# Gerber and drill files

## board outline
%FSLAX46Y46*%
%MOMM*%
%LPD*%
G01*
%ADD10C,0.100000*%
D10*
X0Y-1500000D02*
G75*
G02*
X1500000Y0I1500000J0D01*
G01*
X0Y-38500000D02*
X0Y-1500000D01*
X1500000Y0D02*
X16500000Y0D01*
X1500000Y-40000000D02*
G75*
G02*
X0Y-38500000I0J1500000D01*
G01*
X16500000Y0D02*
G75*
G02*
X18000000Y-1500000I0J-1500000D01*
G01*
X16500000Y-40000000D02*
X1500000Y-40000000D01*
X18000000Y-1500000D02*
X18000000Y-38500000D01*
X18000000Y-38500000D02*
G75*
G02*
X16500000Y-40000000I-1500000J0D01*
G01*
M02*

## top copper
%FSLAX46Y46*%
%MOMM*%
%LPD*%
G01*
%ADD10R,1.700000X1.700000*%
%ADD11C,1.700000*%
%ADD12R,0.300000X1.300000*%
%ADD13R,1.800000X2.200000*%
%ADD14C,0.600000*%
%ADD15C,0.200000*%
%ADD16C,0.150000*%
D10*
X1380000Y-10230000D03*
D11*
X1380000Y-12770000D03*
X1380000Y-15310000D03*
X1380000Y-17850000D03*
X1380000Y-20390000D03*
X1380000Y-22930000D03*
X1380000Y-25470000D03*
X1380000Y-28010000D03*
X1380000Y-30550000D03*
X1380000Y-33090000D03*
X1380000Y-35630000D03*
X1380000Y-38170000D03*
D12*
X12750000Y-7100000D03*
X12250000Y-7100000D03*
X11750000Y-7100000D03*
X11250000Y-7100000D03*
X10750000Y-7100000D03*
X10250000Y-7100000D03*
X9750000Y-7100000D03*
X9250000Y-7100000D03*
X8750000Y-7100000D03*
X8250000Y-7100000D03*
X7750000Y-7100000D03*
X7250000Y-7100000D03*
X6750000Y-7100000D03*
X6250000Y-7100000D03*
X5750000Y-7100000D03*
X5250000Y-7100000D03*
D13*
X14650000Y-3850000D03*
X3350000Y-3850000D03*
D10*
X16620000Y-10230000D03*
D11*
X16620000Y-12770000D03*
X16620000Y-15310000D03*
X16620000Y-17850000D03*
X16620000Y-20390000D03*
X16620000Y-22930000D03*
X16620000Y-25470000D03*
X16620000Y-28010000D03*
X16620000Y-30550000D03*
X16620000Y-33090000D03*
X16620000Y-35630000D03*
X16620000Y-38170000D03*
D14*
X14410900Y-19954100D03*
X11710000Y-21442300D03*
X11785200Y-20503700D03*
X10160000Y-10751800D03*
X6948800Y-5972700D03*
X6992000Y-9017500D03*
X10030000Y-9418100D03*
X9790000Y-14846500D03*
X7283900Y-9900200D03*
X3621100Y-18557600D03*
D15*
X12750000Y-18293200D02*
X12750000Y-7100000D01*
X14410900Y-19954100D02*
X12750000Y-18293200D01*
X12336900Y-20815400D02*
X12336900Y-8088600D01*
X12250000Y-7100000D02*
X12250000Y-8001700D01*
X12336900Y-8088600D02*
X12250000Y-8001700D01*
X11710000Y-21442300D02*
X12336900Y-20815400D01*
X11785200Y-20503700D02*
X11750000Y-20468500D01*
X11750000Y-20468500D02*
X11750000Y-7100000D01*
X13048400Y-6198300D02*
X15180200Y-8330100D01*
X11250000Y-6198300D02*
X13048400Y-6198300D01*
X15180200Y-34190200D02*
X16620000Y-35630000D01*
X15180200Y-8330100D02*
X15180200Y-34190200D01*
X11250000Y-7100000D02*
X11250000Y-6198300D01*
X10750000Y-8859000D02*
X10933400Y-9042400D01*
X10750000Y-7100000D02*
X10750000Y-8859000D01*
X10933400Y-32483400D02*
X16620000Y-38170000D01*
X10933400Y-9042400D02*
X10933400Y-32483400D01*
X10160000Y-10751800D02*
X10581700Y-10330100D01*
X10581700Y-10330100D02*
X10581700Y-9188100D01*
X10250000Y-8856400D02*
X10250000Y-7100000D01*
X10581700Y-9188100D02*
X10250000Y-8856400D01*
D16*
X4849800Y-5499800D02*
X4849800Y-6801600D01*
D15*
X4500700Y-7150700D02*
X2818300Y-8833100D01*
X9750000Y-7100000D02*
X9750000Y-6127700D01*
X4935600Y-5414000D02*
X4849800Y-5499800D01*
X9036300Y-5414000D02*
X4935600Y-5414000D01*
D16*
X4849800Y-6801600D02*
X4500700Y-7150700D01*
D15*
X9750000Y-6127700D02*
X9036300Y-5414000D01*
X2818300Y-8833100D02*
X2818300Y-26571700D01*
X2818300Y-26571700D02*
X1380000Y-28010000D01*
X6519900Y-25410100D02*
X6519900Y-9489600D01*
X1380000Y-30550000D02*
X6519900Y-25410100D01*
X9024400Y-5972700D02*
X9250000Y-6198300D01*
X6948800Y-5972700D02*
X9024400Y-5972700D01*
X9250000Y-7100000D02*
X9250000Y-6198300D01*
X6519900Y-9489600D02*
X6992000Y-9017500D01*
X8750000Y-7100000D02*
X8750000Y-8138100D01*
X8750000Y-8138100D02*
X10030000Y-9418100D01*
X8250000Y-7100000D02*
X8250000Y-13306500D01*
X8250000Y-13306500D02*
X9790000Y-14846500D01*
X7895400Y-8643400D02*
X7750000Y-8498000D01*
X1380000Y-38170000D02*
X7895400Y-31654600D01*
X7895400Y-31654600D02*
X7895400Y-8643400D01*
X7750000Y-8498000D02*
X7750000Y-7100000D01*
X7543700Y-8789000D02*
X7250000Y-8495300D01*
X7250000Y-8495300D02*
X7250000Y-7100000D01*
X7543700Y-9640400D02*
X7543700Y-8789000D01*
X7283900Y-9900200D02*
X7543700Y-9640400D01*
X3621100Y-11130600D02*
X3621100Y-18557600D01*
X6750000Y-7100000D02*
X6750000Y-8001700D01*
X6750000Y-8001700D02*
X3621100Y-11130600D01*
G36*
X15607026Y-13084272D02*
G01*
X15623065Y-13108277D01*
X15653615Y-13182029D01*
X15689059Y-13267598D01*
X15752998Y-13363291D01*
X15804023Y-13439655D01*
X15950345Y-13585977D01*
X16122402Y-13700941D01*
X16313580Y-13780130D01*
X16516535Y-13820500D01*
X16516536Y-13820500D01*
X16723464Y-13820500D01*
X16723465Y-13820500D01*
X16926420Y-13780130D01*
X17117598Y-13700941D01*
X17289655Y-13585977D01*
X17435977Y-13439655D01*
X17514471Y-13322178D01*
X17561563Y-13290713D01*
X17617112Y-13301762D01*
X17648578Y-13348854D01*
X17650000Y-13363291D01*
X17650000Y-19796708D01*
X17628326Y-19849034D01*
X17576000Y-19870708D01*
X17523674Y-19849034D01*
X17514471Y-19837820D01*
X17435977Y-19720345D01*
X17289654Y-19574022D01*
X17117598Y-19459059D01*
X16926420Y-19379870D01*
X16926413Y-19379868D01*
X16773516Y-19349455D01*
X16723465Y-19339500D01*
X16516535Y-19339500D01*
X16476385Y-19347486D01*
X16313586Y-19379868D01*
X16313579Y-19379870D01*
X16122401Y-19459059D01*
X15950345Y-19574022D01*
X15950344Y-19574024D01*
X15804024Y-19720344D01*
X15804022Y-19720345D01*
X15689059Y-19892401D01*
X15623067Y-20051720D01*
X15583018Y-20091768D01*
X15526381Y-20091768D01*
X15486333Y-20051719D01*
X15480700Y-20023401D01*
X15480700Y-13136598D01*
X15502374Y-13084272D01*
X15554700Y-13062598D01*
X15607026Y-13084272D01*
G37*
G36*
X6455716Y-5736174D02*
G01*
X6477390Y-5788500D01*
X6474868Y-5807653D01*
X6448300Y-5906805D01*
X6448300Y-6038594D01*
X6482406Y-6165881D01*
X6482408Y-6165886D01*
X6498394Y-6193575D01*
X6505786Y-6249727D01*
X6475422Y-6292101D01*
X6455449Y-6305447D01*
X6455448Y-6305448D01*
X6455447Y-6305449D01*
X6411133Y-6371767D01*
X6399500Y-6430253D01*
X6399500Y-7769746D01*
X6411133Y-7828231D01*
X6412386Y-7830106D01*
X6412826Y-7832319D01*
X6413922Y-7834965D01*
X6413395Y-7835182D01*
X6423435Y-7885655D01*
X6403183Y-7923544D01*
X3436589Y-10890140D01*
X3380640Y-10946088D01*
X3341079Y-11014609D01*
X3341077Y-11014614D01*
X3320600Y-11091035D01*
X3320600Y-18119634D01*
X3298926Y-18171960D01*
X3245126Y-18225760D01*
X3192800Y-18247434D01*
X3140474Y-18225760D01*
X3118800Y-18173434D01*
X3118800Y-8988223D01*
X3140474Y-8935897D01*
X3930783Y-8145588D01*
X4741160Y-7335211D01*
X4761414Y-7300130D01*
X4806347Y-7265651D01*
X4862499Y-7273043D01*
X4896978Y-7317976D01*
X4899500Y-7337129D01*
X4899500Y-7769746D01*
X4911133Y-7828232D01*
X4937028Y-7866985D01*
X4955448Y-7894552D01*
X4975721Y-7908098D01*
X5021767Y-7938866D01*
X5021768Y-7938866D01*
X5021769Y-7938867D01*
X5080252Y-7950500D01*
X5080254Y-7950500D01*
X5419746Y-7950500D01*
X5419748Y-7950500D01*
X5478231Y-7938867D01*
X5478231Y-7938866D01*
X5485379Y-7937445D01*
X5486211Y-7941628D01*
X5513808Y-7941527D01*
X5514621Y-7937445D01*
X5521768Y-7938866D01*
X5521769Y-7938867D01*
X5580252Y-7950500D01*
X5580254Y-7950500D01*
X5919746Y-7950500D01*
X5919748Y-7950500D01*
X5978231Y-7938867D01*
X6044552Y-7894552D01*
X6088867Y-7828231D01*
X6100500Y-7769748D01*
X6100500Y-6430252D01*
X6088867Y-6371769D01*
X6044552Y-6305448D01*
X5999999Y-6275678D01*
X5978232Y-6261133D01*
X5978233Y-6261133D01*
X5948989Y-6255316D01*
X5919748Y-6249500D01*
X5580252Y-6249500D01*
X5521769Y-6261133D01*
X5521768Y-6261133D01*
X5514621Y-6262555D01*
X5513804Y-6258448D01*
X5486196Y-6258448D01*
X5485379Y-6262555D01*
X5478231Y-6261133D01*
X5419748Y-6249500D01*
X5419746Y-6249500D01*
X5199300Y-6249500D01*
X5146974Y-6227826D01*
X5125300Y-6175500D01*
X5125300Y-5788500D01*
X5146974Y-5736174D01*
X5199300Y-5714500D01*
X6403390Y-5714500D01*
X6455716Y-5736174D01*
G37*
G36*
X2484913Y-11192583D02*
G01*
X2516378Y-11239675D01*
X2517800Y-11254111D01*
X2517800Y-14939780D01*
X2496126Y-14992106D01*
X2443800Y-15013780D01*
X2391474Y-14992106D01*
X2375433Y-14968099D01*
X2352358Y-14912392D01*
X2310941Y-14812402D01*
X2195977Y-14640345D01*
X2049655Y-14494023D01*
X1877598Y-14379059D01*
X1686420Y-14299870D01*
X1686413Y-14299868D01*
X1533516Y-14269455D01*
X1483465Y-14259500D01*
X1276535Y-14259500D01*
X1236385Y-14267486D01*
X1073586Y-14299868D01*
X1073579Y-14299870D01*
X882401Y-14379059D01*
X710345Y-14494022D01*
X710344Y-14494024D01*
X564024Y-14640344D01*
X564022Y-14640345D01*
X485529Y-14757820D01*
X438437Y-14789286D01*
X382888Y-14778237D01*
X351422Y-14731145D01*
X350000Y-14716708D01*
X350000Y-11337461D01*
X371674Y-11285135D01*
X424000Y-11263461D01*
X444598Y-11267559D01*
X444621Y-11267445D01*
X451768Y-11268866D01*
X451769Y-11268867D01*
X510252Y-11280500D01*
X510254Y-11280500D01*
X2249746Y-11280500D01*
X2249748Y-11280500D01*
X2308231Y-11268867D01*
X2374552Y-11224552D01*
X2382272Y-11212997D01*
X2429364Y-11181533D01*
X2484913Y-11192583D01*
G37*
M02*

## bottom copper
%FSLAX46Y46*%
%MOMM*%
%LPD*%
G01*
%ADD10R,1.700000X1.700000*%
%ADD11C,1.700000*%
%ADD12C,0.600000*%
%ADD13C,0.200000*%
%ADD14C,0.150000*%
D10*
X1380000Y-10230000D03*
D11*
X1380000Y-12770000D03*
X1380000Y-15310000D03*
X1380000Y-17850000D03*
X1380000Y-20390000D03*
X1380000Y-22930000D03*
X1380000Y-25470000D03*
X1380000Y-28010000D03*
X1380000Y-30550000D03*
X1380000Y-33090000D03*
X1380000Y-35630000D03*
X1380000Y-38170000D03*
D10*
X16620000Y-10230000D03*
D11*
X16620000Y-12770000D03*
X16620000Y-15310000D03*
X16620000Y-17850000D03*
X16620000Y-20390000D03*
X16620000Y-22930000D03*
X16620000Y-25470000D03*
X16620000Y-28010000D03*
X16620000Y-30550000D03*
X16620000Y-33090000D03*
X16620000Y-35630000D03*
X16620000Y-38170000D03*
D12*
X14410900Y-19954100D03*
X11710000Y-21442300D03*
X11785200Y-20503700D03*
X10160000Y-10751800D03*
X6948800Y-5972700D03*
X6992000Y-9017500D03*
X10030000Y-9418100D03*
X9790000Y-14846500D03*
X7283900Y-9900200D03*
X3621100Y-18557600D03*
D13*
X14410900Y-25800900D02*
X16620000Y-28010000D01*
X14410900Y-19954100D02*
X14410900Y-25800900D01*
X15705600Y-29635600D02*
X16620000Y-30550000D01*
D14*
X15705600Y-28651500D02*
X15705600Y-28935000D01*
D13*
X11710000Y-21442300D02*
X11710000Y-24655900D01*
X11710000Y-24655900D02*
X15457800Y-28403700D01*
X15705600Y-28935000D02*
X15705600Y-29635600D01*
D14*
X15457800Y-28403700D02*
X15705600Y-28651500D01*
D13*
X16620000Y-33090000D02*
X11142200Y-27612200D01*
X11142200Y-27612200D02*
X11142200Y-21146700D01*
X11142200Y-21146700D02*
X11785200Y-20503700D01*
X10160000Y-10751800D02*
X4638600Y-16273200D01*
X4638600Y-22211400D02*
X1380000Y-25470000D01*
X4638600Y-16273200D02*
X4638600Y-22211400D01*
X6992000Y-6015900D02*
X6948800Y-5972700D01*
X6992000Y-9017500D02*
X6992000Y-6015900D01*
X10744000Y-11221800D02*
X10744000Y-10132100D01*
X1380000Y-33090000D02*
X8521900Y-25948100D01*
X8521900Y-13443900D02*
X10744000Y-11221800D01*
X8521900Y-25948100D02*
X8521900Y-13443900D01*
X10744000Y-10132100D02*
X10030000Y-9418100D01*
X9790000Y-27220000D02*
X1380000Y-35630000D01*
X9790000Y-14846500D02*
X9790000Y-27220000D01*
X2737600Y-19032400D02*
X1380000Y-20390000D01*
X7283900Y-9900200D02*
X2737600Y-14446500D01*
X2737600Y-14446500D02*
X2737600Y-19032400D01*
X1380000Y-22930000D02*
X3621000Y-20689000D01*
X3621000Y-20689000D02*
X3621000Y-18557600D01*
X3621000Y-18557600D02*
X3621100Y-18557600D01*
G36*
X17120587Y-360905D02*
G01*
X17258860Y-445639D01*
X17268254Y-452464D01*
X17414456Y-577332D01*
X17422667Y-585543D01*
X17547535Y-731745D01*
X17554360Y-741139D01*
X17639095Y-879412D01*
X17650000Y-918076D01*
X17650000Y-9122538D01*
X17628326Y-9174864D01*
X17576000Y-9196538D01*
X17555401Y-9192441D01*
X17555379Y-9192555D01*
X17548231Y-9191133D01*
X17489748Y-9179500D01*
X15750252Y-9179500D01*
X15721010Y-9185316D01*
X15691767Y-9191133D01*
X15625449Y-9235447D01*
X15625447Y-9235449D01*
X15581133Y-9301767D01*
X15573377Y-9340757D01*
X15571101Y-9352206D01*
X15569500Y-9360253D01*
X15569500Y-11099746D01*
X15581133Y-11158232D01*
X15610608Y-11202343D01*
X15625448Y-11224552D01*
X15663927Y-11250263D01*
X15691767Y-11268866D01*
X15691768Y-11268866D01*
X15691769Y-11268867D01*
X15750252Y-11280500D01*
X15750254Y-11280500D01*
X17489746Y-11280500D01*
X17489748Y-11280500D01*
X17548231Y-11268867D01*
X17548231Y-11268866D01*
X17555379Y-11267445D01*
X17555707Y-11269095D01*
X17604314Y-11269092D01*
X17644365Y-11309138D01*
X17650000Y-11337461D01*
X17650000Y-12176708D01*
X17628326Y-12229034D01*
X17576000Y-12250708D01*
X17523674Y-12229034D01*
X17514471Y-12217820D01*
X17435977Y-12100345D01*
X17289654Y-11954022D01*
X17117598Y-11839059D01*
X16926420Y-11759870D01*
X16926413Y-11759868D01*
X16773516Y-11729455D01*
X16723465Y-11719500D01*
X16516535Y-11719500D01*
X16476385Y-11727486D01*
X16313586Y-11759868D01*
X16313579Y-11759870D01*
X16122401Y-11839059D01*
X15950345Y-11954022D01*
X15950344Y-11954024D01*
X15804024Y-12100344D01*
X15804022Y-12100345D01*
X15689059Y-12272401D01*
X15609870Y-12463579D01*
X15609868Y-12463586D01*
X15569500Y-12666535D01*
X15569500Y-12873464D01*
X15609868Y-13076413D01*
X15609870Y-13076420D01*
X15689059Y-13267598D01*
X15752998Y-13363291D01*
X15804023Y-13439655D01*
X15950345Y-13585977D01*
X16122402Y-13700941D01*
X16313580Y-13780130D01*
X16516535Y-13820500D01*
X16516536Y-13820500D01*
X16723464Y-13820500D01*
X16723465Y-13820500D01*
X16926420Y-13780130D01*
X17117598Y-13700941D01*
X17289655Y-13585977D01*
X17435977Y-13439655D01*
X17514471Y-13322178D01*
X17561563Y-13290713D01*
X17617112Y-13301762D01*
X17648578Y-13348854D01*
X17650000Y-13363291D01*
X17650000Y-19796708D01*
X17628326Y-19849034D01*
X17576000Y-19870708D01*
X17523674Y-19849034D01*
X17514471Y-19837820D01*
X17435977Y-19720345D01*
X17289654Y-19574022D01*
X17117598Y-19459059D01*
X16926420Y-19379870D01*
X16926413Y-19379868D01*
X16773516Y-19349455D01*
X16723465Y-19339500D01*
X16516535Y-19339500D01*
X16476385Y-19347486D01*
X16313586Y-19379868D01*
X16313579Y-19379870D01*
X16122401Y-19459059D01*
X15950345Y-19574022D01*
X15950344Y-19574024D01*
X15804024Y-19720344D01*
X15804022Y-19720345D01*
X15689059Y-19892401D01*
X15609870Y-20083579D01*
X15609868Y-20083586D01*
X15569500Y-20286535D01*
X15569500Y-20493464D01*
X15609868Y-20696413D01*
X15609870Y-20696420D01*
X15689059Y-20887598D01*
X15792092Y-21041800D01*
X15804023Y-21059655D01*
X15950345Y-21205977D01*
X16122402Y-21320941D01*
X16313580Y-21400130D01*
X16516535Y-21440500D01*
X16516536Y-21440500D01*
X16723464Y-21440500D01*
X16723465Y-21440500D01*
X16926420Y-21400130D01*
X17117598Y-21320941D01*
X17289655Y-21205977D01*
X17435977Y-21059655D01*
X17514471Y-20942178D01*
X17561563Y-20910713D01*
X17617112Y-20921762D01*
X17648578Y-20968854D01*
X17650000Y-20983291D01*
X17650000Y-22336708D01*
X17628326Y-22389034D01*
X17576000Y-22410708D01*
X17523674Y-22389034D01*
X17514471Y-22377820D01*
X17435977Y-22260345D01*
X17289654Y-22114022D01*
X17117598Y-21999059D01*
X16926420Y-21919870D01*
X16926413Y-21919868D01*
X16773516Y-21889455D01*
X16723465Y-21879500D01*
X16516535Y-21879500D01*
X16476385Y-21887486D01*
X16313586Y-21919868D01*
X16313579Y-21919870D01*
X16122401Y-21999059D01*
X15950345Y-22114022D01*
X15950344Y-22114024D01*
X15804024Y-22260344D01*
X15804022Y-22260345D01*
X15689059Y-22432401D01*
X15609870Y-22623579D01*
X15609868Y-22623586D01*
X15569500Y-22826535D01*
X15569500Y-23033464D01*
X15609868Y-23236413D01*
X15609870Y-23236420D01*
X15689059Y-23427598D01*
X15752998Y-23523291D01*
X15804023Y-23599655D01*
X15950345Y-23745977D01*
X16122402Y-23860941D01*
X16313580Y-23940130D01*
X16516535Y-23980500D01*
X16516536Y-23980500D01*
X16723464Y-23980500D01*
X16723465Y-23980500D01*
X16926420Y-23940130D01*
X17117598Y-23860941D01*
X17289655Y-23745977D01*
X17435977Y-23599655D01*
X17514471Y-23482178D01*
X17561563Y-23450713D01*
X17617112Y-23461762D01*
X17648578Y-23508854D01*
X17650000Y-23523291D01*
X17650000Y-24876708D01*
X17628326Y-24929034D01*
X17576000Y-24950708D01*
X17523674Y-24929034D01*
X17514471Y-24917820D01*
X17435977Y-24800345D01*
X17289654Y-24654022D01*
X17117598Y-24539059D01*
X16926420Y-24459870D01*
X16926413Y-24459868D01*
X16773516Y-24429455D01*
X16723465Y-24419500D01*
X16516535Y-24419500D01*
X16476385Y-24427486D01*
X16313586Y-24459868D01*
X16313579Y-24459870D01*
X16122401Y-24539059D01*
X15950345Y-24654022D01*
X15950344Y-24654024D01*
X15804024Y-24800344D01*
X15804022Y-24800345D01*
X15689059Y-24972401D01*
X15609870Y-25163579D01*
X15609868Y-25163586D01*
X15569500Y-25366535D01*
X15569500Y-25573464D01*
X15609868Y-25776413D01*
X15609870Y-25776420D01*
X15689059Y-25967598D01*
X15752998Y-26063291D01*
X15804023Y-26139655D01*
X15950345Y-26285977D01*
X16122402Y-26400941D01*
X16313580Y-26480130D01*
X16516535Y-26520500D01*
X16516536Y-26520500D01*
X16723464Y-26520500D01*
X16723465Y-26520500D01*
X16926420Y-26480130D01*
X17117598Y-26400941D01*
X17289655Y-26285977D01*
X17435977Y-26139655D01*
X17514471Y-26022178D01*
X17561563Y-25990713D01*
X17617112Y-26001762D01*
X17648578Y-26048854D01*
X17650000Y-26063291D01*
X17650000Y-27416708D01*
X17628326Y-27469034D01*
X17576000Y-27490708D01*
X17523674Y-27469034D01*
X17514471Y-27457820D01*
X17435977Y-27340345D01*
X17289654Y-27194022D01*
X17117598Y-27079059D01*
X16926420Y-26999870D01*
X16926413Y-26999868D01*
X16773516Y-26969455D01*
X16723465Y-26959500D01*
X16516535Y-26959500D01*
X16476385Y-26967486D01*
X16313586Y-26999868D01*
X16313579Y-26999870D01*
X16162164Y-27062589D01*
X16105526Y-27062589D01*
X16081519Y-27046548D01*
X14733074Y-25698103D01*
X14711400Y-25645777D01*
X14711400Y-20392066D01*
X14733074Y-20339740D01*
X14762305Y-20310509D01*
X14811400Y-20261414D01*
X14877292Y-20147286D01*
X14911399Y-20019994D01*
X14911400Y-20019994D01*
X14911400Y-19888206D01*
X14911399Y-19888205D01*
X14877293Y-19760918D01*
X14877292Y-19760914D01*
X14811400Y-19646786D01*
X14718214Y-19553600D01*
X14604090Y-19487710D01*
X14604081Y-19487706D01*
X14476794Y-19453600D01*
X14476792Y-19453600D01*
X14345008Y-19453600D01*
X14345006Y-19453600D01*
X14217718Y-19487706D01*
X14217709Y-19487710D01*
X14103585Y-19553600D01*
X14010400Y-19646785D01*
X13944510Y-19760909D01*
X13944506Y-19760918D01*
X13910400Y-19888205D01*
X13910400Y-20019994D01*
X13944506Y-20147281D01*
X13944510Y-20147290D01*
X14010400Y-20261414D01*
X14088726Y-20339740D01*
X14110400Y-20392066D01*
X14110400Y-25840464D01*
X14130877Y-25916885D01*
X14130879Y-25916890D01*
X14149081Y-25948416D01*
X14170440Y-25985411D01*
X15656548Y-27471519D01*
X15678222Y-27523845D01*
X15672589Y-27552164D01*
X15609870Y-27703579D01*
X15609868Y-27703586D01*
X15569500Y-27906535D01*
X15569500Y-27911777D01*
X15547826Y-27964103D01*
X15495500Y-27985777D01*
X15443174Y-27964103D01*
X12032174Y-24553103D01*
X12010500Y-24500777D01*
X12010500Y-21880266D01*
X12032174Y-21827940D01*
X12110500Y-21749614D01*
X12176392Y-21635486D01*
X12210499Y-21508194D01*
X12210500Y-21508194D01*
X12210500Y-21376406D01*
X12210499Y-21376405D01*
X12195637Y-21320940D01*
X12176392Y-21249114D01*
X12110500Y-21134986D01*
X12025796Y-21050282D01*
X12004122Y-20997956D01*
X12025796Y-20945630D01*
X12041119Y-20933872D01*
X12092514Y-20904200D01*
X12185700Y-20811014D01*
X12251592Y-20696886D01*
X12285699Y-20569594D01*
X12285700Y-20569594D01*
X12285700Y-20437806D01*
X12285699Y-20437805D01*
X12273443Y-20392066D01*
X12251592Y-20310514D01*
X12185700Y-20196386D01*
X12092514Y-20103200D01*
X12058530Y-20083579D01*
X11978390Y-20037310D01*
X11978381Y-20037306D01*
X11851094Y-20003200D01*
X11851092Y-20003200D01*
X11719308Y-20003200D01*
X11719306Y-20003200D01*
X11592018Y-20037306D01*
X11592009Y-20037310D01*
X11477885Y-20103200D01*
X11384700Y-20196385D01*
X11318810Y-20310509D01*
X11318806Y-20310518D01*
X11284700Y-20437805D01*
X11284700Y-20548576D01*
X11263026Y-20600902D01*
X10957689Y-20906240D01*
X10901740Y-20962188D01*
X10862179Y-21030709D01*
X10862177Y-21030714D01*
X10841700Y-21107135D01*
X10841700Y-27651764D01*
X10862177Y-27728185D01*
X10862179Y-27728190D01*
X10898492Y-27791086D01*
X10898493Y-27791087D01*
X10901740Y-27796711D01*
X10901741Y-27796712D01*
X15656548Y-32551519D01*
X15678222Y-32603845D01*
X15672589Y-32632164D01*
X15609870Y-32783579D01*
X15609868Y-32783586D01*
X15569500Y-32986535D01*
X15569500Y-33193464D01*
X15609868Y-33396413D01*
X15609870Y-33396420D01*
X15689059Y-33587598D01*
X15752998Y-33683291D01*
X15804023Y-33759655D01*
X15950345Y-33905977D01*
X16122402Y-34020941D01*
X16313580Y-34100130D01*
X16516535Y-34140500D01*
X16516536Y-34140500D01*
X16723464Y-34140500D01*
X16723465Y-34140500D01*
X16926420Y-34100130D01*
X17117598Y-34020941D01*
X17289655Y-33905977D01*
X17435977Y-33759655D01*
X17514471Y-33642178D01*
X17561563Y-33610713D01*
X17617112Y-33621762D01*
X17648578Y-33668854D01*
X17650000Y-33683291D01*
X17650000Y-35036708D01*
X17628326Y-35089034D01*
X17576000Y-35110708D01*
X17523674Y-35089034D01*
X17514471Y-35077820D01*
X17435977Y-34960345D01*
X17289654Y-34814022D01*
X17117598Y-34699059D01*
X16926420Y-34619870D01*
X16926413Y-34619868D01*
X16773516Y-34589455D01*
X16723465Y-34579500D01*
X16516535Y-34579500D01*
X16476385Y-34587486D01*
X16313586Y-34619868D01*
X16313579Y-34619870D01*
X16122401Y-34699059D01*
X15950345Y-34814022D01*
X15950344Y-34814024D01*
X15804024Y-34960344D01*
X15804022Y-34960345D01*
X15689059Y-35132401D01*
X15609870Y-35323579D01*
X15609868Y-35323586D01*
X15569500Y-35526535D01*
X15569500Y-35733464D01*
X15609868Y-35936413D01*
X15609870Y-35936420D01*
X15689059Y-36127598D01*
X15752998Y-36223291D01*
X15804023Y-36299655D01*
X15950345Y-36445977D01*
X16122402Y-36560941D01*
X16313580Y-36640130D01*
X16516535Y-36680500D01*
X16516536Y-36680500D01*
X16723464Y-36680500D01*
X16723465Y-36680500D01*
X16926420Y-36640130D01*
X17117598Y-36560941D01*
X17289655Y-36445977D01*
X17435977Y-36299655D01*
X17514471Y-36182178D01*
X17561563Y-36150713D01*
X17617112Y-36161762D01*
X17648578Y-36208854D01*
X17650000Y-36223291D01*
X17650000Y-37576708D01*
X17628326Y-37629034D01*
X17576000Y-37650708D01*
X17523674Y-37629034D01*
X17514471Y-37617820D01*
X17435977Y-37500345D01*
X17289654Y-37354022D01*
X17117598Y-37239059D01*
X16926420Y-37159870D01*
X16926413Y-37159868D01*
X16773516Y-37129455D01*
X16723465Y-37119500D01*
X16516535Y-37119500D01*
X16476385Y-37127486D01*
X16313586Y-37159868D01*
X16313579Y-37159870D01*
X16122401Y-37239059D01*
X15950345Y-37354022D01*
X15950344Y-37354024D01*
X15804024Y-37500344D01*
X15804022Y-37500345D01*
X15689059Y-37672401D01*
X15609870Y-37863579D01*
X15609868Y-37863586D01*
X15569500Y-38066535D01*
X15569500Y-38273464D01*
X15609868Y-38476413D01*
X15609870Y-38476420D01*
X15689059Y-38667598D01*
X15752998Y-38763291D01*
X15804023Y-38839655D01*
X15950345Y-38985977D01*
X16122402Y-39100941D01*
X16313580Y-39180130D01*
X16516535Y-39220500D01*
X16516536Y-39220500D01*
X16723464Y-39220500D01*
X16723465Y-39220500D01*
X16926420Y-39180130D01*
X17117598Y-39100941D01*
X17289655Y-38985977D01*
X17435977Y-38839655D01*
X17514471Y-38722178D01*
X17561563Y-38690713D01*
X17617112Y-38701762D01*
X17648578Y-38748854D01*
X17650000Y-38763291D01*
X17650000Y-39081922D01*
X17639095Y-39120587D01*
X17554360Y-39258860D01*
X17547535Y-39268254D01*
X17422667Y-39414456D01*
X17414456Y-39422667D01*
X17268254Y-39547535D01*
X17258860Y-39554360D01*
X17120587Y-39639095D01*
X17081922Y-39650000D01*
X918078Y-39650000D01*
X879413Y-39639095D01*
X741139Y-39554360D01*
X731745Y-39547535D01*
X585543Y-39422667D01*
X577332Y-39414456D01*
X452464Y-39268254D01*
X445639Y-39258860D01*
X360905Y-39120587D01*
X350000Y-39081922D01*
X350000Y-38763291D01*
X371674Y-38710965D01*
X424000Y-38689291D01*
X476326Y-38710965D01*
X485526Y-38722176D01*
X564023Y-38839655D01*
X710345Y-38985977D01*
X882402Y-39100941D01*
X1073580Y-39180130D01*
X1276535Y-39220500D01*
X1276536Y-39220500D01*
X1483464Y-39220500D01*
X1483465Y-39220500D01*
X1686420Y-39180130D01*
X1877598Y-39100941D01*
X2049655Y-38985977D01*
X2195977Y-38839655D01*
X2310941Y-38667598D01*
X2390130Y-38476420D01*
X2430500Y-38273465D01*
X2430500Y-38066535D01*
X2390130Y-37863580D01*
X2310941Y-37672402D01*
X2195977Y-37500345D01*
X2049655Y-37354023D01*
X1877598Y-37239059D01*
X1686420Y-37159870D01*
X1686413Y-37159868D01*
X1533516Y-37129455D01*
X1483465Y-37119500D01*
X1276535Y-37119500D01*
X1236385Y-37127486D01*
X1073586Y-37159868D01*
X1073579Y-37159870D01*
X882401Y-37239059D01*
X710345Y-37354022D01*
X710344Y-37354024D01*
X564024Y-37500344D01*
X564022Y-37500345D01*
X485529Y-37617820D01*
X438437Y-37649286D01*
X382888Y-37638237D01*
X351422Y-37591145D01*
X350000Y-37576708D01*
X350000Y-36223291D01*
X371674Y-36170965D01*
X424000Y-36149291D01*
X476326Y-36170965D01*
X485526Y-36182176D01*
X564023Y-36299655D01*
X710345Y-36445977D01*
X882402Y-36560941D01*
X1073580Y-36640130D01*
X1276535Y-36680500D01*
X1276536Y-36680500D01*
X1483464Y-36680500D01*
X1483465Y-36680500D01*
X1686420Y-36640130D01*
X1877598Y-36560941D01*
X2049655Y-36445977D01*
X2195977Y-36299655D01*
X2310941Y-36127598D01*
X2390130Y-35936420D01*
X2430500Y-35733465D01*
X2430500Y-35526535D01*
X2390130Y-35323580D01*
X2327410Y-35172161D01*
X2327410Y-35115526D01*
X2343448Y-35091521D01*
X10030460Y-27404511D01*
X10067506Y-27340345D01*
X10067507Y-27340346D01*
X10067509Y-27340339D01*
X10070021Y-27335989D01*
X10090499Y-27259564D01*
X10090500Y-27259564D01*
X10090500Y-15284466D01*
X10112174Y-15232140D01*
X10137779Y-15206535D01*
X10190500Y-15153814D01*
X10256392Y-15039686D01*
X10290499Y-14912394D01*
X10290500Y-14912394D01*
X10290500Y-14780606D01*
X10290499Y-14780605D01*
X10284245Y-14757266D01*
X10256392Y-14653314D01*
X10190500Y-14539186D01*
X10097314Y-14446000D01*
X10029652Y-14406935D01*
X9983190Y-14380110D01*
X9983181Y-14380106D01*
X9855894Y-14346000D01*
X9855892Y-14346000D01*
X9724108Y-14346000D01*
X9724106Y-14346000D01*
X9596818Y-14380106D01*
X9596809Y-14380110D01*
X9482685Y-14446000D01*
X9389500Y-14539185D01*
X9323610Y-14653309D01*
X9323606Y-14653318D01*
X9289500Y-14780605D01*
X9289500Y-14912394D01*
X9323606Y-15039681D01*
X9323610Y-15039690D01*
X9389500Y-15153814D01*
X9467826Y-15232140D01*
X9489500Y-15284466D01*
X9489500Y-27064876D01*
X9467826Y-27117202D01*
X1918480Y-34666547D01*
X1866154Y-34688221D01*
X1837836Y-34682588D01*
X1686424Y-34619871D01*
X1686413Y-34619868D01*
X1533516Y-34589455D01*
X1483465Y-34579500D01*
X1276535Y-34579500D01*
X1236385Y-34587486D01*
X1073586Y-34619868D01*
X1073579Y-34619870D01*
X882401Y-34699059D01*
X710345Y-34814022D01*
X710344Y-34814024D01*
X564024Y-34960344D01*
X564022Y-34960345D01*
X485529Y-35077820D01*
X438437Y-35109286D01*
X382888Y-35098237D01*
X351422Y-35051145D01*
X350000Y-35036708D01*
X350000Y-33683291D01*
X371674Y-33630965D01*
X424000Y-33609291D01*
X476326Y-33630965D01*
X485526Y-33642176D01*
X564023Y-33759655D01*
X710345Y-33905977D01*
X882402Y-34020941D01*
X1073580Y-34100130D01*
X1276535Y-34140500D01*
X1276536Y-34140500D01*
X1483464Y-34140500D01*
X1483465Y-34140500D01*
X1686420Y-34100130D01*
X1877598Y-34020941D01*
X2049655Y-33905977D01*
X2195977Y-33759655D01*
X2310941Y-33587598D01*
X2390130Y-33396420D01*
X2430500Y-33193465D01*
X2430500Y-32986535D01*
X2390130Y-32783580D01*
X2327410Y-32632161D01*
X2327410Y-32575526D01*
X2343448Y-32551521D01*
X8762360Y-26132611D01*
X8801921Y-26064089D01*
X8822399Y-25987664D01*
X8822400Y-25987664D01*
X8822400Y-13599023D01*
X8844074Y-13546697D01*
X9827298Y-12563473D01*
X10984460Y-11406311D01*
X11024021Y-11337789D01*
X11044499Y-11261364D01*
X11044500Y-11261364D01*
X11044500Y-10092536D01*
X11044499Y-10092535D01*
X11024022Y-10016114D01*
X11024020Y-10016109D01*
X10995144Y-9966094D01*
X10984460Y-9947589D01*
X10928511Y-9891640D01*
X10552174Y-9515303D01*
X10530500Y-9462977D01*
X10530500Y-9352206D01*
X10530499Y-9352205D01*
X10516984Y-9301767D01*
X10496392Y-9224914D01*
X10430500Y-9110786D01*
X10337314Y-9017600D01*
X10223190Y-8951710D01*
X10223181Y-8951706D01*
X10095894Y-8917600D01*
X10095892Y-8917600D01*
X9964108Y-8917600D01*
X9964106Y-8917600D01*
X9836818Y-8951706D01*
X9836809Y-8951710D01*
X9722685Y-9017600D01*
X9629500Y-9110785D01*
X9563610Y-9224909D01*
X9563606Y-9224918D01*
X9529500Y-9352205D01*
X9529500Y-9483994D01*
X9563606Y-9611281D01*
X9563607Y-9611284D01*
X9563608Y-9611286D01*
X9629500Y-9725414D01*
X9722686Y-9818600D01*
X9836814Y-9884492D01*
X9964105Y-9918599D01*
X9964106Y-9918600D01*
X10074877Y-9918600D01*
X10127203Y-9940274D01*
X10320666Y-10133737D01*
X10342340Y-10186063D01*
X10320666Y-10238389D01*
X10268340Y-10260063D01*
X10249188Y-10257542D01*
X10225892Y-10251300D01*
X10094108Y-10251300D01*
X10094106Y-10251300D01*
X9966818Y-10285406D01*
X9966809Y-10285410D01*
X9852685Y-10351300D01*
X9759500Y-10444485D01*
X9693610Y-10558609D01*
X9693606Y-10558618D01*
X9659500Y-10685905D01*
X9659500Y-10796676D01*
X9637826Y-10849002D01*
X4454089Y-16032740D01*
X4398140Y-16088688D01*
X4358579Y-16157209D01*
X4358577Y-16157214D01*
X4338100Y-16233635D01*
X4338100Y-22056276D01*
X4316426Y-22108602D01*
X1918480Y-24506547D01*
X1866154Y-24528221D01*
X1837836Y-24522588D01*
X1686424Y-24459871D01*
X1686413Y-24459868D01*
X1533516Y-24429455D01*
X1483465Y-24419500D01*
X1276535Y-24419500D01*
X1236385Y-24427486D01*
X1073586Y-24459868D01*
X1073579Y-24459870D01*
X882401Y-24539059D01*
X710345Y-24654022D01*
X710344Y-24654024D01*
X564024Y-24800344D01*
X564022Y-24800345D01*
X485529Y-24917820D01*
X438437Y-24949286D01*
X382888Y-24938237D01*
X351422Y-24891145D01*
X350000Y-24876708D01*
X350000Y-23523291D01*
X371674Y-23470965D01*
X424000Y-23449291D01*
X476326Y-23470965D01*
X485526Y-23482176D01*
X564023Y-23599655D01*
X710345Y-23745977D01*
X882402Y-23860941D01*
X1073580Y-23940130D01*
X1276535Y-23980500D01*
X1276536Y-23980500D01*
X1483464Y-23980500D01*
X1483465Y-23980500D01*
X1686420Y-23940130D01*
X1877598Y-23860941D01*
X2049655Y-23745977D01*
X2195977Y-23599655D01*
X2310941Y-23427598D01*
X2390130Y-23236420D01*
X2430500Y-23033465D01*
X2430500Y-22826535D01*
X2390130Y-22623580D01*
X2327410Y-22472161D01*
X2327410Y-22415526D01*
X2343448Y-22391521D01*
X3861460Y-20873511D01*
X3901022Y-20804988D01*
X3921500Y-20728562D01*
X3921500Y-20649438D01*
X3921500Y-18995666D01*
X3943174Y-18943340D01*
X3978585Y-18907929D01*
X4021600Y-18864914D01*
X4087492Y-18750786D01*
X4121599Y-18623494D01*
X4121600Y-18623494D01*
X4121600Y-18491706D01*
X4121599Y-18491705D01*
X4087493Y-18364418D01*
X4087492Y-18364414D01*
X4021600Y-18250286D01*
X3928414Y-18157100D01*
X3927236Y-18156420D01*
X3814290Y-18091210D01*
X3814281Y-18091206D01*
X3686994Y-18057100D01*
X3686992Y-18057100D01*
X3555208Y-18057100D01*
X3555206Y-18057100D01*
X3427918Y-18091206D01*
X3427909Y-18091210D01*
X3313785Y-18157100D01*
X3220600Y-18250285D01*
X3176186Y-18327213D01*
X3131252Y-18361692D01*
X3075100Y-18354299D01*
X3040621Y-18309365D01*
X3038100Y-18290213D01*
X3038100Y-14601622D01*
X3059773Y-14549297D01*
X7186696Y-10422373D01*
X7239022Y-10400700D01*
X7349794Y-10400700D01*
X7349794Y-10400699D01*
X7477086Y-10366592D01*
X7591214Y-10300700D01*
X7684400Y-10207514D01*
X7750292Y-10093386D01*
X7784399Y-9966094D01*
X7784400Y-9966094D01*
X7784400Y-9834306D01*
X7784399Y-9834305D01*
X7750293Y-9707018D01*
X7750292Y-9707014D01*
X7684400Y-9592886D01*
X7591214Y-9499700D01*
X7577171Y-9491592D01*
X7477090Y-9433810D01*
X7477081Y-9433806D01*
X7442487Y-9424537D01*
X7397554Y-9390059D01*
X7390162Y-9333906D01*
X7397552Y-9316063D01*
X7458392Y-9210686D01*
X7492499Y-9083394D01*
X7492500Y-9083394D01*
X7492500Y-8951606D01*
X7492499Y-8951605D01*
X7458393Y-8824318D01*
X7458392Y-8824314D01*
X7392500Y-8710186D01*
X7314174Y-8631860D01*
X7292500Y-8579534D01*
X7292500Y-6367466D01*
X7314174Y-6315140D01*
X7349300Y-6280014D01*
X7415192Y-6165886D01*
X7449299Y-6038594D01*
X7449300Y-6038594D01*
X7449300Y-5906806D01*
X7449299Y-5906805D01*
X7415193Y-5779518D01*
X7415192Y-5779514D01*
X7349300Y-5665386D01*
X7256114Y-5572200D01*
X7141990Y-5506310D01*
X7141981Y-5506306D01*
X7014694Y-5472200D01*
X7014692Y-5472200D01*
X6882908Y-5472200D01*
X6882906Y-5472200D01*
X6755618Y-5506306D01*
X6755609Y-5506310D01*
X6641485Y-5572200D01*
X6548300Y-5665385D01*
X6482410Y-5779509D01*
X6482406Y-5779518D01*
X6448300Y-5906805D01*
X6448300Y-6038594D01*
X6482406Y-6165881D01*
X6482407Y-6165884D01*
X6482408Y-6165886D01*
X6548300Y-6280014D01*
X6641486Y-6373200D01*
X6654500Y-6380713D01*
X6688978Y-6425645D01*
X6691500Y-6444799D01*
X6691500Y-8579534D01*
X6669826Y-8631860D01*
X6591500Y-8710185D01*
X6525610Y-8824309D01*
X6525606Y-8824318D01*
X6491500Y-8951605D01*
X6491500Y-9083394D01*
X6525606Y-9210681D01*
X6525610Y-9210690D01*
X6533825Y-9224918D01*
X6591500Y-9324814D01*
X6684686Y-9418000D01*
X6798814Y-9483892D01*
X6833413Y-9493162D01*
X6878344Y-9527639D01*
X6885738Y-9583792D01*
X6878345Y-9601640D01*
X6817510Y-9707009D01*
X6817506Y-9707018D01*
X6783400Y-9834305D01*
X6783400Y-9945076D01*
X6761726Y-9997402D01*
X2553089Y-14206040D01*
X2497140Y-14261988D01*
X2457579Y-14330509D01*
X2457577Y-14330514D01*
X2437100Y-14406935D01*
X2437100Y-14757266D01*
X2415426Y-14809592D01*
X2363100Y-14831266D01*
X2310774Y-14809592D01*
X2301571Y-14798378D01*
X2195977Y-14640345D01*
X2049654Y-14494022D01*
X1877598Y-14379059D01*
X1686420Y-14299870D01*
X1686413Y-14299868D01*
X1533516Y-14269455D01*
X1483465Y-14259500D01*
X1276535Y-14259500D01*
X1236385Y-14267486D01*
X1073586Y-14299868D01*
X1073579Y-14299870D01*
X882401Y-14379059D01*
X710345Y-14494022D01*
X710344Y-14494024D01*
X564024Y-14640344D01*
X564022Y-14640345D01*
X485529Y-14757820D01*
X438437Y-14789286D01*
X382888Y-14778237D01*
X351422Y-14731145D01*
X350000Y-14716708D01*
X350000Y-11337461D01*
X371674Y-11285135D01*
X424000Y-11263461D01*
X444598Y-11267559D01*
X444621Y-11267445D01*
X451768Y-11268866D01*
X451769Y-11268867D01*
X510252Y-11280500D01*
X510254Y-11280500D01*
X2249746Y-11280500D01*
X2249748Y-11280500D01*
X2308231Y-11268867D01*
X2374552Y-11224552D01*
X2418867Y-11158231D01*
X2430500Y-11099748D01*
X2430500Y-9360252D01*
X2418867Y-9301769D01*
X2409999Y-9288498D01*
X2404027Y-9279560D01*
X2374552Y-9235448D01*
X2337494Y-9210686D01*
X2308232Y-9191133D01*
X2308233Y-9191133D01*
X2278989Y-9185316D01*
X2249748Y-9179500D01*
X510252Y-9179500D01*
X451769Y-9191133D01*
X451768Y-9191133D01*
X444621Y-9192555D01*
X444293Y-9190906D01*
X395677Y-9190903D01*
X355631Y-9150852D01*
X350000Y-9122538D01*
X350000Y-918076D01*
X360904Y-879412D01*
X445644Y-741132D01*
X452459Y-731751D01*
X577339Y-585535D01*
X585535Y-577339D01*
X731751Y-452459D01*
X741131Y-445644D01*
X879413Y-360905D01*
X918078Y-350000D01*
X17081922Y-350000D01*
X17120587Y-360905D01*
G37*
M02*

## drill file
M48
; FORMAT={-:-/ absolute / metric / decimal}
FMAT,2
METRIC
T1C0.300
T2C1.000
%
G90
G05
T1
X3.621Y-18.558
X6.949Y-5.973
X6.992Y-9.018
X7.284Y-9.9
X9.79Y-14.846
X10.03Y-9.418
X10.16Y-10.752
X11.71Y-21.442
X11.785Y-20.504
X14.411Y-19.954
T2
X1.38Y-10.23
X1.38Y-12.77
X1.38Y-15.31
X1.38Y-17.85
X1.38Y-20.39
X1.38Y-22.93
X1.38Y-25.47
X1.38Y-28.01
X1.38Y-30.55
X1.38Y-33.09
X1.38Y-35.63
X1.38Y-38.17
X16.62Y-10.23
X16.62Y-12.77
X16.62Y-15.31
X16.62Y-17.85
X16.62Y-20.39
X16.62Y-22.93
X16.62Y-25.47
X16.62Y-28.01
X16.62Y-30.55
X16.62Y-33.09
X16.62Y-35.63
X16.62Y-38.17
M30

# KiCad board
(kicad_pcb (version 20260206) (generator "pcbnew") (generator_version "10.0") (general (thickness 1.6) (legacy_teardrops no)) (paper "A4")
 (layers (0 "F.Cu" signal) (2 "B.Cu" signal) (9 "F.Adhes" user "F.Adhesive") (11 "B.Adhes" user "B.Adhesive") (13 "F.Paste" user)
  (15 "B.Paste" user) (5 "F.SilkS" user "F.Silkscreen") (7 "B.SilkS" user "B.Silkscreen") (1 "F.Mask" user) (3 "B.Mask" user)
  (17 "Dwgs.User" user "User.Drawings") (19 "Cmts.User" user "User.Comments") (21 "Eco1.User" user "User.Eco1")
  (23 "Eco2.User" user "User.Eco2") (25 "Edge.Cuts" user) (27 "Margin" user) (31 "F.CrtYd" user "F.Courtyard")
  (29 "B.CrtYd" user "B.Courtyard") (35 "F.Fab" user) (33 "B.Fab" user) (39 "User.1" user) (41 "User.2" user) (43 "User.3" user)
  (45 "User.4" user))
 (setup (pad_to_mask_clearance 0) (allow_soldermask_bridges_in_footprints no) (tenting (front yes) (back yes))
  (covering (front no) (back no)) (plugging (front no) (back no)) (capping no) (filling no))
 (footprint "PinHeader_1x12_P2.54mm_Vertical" (layer "F.Cu") (at 1.38 10.23)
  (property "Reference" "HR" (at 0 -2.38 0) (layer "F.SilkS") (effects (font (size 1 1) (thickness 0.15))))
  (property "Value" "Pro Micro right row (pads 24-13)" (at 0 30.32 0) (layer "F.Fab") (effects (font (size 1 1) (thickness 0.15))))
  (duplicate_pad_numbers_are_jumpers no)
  (pad "1" thru_hole rect (at 0 0) (size 1.7 1.7) (drill 1) (layers "*.Cu" "*.Mask") (remove_unused_layers no))
  (pad "2" thru_hole circle (at 0 2.54) (size 1.7 1.7) (drill 1) (layers "*.Cu" "*.Mask") (remove_unused_layers no) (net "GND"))
  (pad "3" thru_hole circle (at 0 5.08) (size 1.7 1.7) (drill 1) (layers "*.Cu" "*.Mask") (remove_unused_layers no))
  (pad "4" thru_hole circle (at 0 7.62) (size 1.7 1.7) (drill 1) (layers "*.Cu" "*.Mask") (remove_unused_layers no))
  (pad "5" thru_hole circle (at 0 10.16) (size 1.7 1.7) (drill 1) (layers "*.Cu" "*.Mask") (remove_unused_layers no) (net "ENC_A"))
  (pad "6" thru_hole circle (at 0 12.7) (size 1.7 1.7) (drill 1) (layers "*.Cu" "*.Mask") (remove_unused_layers no) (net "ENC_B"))
  (pad "7" thru_hole circle (at 0 15.24) (size 1.7 1.7) (drill 1) (layers "*.Cu" "*.Mask") (remove_unused_layers no) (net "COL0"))
  (pad "8" thru_hole circle (at 0 17.78) (size 1.7 1.7) (drill 1) (layers "*.Cu" "*.Mask") (remove_unused_layers no) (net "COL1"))
  (pad "9" thru_hole circle (at 0 20.32) (size 1.7 1.7) (drill 1) (layers "*.Cu" "*.Mask") (remove_unused_layers no) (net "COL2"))
  (pad "10" thru_hole circle (at 0 22.86) (size 1.7 1.7) (drill 1) (layers "*.Cu" "*.Mask") (remove_unused_layers no) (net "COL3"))
  (pad "11" thru_hole circle (at 0 25.4) (size 1.7 1.7) (drill 1) (layers "*.Cu" "*.Mask") (remove_unused_layers no) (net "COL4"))
  (pad "12" thru_hole circle (at 0 27.94) (size 1.7 1.7) (drill 1) (layers "*.Cu" "*.Mask") (remove_unused_layers no) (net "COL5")))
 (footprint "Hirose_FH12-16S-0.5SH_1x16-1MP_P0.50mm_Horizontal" (layer "F.Cu") (at 9 5.25 180)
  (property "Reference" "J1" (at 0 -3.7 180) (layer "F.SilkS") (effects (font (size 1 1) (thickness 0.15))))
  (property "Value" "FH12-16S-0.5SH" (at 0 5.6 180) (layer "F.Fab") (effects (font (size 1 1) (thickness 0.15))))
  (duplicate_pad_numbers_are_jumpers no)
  (pad "1" smd rect (at -3.75 -1.85 180) (size 0.3 1.3) (layers "F.Cu" "F.Mask" "F.Paste") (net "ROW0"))
  (pad "2" smd rect (at -3.25 -1.85 180) (size 0.3 1.3) (layers "F.Cu" "F.Mask" "F.Paste") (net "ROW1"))
  (pad "3" smd rect (at -2.75 -1.85 180) (size 0.3 1.3) (layers "F.Cu" "F.Mask" "F.Paste") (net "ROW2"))
  (pad "4" smd rect (at -2.25 -1.85 180) (size 0.3 1.3) (layers "F.Cu" "F.Mask" "F.Paste") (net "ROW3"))
  (pad "5" smd rect (at -1.75 -1.85 180) (size 0.3 1.3) (layers "F.Cu" "F.Mask" "F.Paste") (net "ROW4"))
  (pad "6" smd rect (at -1.25 -1.85 180) (size 0.3 1.3) (layers "F.Cu" "F.Mask" "F.Paste") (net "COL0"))
  (pad "7" smd rect (at -0.75 -1.85 180) (size 0.3 1.3) (layers "F.Cu" "F.Mask" "F.Paste") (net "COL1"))
  (pad "8" smd rect (at -0.25 -1.85 180) (size 0.3 1.3) (layers "F.Cu" "F.Mask" "F.Paste") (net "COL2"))
  (pad "9" smd rect (at 0.25 -1.85 180) (size 0.3 1.3) (layers "F.Cu" "F.Mask" "F.Paste") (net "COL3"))
  (pad "10" smd rect (at 0.75 -1.85 180) (size 0.3 1.3) (layers "F.Cu" "F.Mask" "F.Paste") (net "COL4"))
  (pad "11" smd rect (at 1.25 -1.85 180) (size 0.3 1.3) (layers "F.Cu" "F.Mask" "F.Paste") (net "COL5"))
  (pad "12" smd rect (at 1.75 -1.85 180) (size 0.3 1.3) (layers "F.Cu" "F.Mask" "F.Paste") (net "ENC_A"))
  (pad "13" smd rect (at 2.25 -1.85 180) (size 0.3 1.3) (layers "F.Cu" "F.Mask" "F.Paste") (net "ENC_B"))
  (pad "14" smd rect (at 2.75 -1.85 180) (size 0.3 1.3) (layers "F.Cu" "F.Mask" "F.Paste") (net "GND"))
  (pad "15" smd rect (at 3.25 -1.85 180) (size 0.3 1.3) (layers "F.Cu" "F.Mask" "F.Paste"))
  (pad "16" smd rect (at 3.75 -1.85 180) (size 0.3 1.3) (layers "F.Cu" "F.Mask" "F.Paste"))
  (pad "MP" smd rect (at -5.65 1.4 180) (size 1.8 2.2) (layers "F.Cu" "F.Mask" "F.Paste"))
  (pad "MP" smd rect (at 5.65 1.4 180) (size 1.8 2.2) (layers "F.Cu" "F.Mask" "F.Paste")))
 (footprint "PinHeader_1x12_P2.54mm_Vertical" (layer "F.Cu") (at 16.62 10.23)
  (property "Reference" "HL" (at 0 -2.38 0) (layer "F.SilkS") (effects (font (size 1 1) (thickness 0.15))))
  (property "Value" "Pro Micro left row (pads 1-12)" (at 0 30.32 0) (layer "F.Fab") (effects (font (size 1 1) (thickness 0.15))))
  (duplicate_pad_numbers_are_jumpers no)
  (pad "1" thru_hole rect (at 0 0) (size 1.7 1.7) (drill 1) (layers "*.Cu" "*.Mask") (remove_unused_layers no))
  (pad "2" thru_hole circle (at 0 2.54) (size 1.7 1.7) (drill 1) (layers "*.Cu" "*.Mask") (remove_unused_layers no))
  (pad "3" thru_hole circle (at 0 5.08) (size 1.7 1.7) (drill 1) (layers "*.Cu" "*.Mask") (remove_unused_layers no) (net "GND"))
  (pad "4" thru_hole circle (at 0 7.62) (size 1.7 1.7) (drill 1) (layers "*.Cu" "*.Mask") (remove_unused_layers no) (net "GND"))
  (pad "5" thru_hole circle (at 0 10.16) (size 1.7 1.7) (drill 1) (layers "*.Cu" "*.Mask") (remove_unused_layers no))
  (pad "6" thru_hole circle (at 0 12.7) (size 1.7 1.7) (drill 1) (layers "*.Cu" "*.Mask") (remove_unused_layers no))
  (pad "7" thru_hole circle (at 0 15.24) (size 1.7 1.7) (drill 1) (layers "*.Cu" "*.Mask") (remove_unused_layers no))
  (pad "8" thru_hole circle (at 0 17.78) (size 1.7 1.7) (drill 1) (layers "*.Cu" "*.Mask") (remove_unused_layers no) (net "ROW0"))
  (pad "9" thru_hole circle (at 0 20.32) (size 1.7 1.7) (drill 1) (layers "*.Cu" "*.Mask") (remove_unused_layers no) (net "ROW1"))
  (pad "10" thru_hole circle (at 0 22.86) (size 1.7 1.7) (drill 1) (layers "*.Cu" "*.Mask") (remove_unused_layers no) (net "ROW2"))
  (pad "11" thru_hole circle (at 0 25.4) (size 1.7 1.7) (drill 1) (layers "*.Cu" "*.Mask") (remove_unused_layers no) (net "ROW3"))
  (pad "12" thru_hole circle (at 0 27.94) (size 1.7 1.7) (drill 1) (layers "*.Cu" "*.Mask") (remove_unused_layers no) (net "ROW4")))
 (gr_arc (start 0 1.5) (mid 0.43934 0.43934) (end 1.5 0) (stroke (width 0.1) (type default)) (layer "Edge.Cuts"))
 (gr_line (start 0 38.5) (end 0 1.5) (stroke (width 0.1) (type default)) (layer "Edge.Cuts"))
 (gr_line (start 1.5 0) (end 16.5 0) (stroke (width 0.1) (type default)) (layer "Edge.Cuts"))
 (gr_arc (start 1.5 40) (mid 0.43934 39.56066) (end 0 38.5) (stroke (width 0.1) (type default)) (layer "Edge.Cuts"))
 (gr_arc (start 16.5 0) (mid 17.56066 0.43934) (end 18 1.5) (stroke (width 0.1) (type default)) (layer "Edge.Cuts"))
 (gr_line (start 16.5 40) (end 1.5 40) (stroke (width 0.1) (type default)) (layer "Edge.Cuts"))
 (gr_line (start 18 1.5) (end 18 38.5) (stroke (width 0.1) (type default)) (layer "Edge.Cuts"))
 (gr_arc (start 18 38.5) (mid 17.56066 39.56066) (end 16.5 40) (stroke (width 0.1) (type default)) (layer "Edge.Cuts"))
 (segment (start 12.75 18.2932) (end 12.75 7.1) (width 0.2) (layer "F.Cu") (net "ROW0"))
 (segment (start 14.4109 19.9541) (end 12.75 18.2932) (width 0.2) (layer "F.Cu") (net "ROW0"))
 (via (at 14.4109 19.9541) (size 0.6) (drill 0.3) (layers "F.Cu" "B.Cu") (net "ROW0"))
 (segment (start 14.4109 25.8009) (end 16.62 28.01) (width 0.2) (layer "B.Cu") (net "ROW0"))
 (segment (start 14.4109 19.9541) (end 14.4109 25.8009) (width 0.2) (layer "B.Cu") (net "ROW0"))
 (segment (start 12.3369 20.8154) (end 12.3369 8.0886) (width 0.2) (layer "F.Cu") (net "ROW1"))
 (segment (start 12.25 7.1) (end 12.25 8.0017) (width 0.2) (layer "F.Cu") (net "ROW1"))
 (segment (start 12.3369 8.0886) (end 12.25 8.0017) (width 0.2) (layer "F.Cu") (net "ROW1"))
 (segment (start 11.71 21.4423) (end 12.3369 20.8154) (width 0.2) (layer "F.Cu") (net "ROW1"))
 (via (at 11.71 21.4423) (size 0.6) (drill 0.3) (layers "F.Cu" "B.Cu") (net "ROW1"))
 (segment (start 15.7056 29.6356) (end 16.62 30.55) (width 0.2) (layer "B.Cu") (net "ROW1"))
 (segment (start 15.7056 28.6515) (end 15.7056 28.935) (width 0.15) (layer "B.Cu") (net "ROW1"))
 (segment (start 11.71 21.4423) (end 11.71 24.6559) (width 0.2) (layer "B.Cu") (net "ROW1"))
 (segment (start 11.71 24.6559) (end 15.4578 28.4037) (width 0.2) (layer "B.Cu") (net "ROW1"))
 (segment (start 15.7056 28.935) (end 15.7056 29.6356) (width 0.2) (layer "B.Cu") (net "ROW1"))
 (segment (start 15.4578 28.4037) (end 15.7056 28.6515) (width 0.15) (layer "B.Cu") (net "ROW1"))
 (segment (start 11.7852 20.5037) (end 11.75 20.4685) (width 0.2) (layer "F.Cu") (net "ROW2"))
 (segment (start 11.75 20.4685) (end 11.75 7.1) (width 0.2) (layer "F.Cu") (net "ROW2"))
 (via (at 11.7852 20.5037) (size 0.6) (drill 0.3) (layers "F.Cu" "B.Cu") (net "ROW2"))
 (segment (start 16.62 33.09) (end 11.1422 27.6122) (width 0.2) (layer "B.Cu") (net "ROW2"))
 (segment (start 11.1422 27.6122) (end 11.1422 21.1467) (width 0.2) (layer "B.Cu") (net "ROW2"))
 (segment (start 11.1422 21.1467) (end 11.7852 20.5037) (width 0.2) (layer "B.Cu") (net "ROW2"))
 (segment (start 13.0484 6.1983) (end 15.1802 8.3301) (width 0.2) (layer "F.Cu") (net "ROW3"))
 (segment (start 11.25 6.1983) (end 13.0484 6.1983) (width 0.2) (layer "F.Cu") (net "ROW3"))
 (segment (start 15.1802 34.1902) (end 16.62 35.63) (width 0.2) (layer "F.Cu") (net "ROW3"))
 (segment (start 15.1802 8.3301) (end 15.1802 34.1902) (width 0.2) (layer "F.Cu") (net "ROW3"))
 (segment (start 11.25 7.1) (end 11.25 6.1983) (width 0.2) (layer "F.Cu") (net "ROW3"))
 (segment (start 10.75 8.859) (end 10.9334 9.0424) (width 0.2) (layer "F.Cu") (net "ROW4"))
 (segment (start 10.75 7.1) (end 10.75 8.859) (width 0.2) (layer "F.Cu") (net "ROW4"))
 (segment (start 10.9334 32.4834) (end 16.62 38.17) (width 0.2) (layer "F.Cu") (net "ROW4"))
 (segment (start 10.9334 9.0424) (end 10.9334 32.4834) (width 0.2) (layer "F.Cu") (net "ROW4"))
 (segment (start 10.16 10.7518) (end 10.5817 10.3301) (width 0.2) (layer "F.Cu") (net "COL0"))
 (segment (start 10.5817 10.3301) (end 10.5817 9.1881) (width 0.2) (layer "F.Cu") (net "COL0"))
 (segment (start 10.25 8.8564) (end 10.25 7.1) (width 0.2) (layer "F.Cu") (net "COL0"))
 (segment (start 10.5817 9.1881) (end 10.25 8.8564) (width 0.2) (layer "F.Cu") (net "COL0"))
 (via (at 10.16 10.7518) (size 0.6) (drill 0.3) (layers "F.Cu" "B.Cu") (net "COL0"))
 (segment (start 10.16 10.7518) (end 4.6386 16.2732) (width 0.2) (layer "B.Cu") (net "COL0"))
 (segment (start 4.6386 22.2114) (end 1.38 25.47) (width 0.2) (layer "B.Cu") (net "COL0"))
 (segment (start 4.6386 16.2732) (end 4.6386 22.2114) (width 0.2) (layer "B.Cu") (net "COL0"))
 (segment (start 4.8498 5.4998) (end 4.8498 6.8016) (width 0.15) (layer "F.Cu") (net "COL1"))
 (segment (start 4.5007 7.1507) (end 2.8183 8.8331) (width 0.2) (layer "F.Cu") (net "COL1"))
 (segment (start 9.75 7.1) (end 9.75 6.1277) (width 0.2) (layer "F.Cu") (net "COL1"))
 (segment (start 4.9356 5.414) (end 4.8498 5.4998) (width 0.2) (layer "F.Cu") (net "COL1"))
 (segment (start 9.0363 5.414) (end 4.9356 5.414) (width 0.2) (layer "F.Cu") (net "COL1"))
 (segment (start 4.8498 6.8016) (end 4.5007 7.1507) (width 0.15) (layer "F.Cu") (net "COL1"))
 (segment (start 9.75 6.1277) (end 9.0363 5.414) (width 0.2) (layer "F.Cu") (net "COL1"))
 (segment (start 2.8183 8.8331) (end 2.8183 26.5717) (width 0.2) (layer "F.Cu") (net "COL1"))
 (segment (start 2.8183 26.5717) (end 1.38 28.01) (width 0.2) (layer "F.Cu") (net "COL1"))
 (segment (start 6.5199 25.4101) (end 6.5199 9.4896) (width 0.2) (layer "F.Cu") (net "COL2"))
 (segment (start 1.38 30.55) (end 6.5199 25.4101) (width 0.2) (layer "F.Cu") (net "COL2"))
 (segment (start 9.0244 5.9727) (end 9.25 6.1983) (width 0.2) (layer "F.Cu") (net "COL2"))
 (segment (start 6.9488 5.9727) (end 9.0244 5.9727) (width 0.2) (layer "F.Cu") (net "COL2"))
 (segment (start 9.25 7.1) (end 9.25 6.1983) (width 0.2) (layer "F.Cu") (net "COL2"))
 (segment (start 6.5199 9.4896) (end 6.992 9.0175) (width 0.2) (layer "F.Cu") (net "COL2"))
 (via (at 6.9488 5.9727) (size 0.6) (drill 0.3) (layers "F.Cu" "B.Cu") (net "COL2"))
 (via (at 6.992 9.0175) (size 0.6) (drill 0.3) (layers "F.Cu" "B.Cu") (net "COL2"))
 (segment (start 6.992 6.0159) (end 6.9488 5.9727) (width 0.2) (layer "B.Cu") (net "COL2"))
 (segment (start 6.992 9.0175) (end 6.992 6.0159) (width 0.2) (layer "B.Cu") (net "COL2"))
 (segment (start 8.75 7.1) (end 8.75 8.1381) (width 0.2) (layer "F.Cu") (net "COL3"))
 (segment (start 8.75 8.1381) (end 10.03 9.4181) (width 0.2) (layer "F.Cu") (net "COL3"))
 (via (at 10.03 9.4181) (size 0.6) (drill 0.3) (layers "F.Cu" "B.Cu") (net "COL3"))
 (segment (start 10.744 11.2218) (end 10.744 10.1321) (width 0.2) (layer "B.Cu") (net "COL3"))
 (segment (start 1.38 33.09) (end 8.5219 25.9481) (width 0.2) (layer "B.Cu") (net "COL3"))
 (segment (start 8.5219 13.4439) (end 10.744 11.2218) (width 0.2) (layer "B.Cu") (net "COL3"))
 (segment (start 8.5219 25.9481) (end 8.5219 13.4439) (width 0.2) (layer "B.Cu") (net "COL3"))
 (segment (start 10.744 10.1321) (end 10.03 9.4181) (width 0.2) (layer "B.Cu") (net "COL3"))
 (segment (start 8.25 7.1) (end 8.25 13.3065) (width 0.2) (layer "F.Cu") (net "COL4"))
 (segment (start 8.25 13.3065) (end 9.79 14.8465) (width 0.2) (layer "F.Cu") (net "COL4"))
 (via (at 9.79 14.8465) (size 0.6) (drill 0.3) (layers "F.Cu" "B.Cu") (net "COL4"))
 (segment (start 9.79 27.22) (end 1.38 35.63) (width 0.2) (layer "B.Cu") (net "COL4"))
 (segment (start 9.79 14.8465) (end 9.79 27.22) (width 0.2) (layer "B.Cu") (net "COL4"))
 (segment (start 7.8954 8.6434) (end 7.75 8.498) (width 0.2) (layer "F.Cu") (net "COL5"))
 (segment (start 1.38 38.17) (end 7.8954 31.6546) (width 0.2) (layer "F.Cu") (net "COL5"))
 (segment (start 7.8954 31.6546) (end 7.8954 8.6434) (width 0.2) (layer "F.Cu") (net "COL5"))
 (segment (start 7.75 8.498) (end 7.75 7.1) (width 0.2) (layer "F.Cu") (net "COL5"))
 (segment (start 7.5437 8.789) (end 7.25 8.4953) (width 0.2) (layer "F.Cu") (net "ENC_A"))
 (segment (start 7.25 8.4953) (end 7.25 7.1) (width 0.2) (layer "F.Cu") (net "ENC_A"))
 (segment (start 7.5437 9.6404) (end 7.5437 8.789) (width 0.2) (layer "F.Cu") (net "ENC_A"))
 (segment (start 7.2839 9.9002) (end 7.5437 9.6404) (width 0.2) (layer "F.Cu") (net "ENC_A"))
 (via (at 7.2839 9.9002) (size 0.6) (drill 0.3) (layers "F.Cu" "B.Cu") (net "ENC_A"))
 (segment (start 2.7376 19.0324) (end 1.38 20.39) (width 0.2) (layer "B.Cu") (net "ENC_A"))
 (segment (start 7.2839 9.9002) (end 2.7376 14.4465) (width 0.2) (layer "B.Cu") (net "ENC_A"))
 (segment (start 2.7376 14.4465) (end 2.7376 19.0324) (width 0.2) (layer "B.Cu") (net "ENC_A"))
 (segment (start 3.6211 11.1306) (end 3.6211 18.5576) (width 0.2) (layer "F.Cu") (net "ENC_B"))
 (segment (start 6.75 7.1) (end 6.75 8.0017) (width 0.2) (layer "F.Cu") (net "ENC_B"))
 (segment (start 6.75 8.0017) (end 3.6211 11.1306) (width 0.2) (layer "F.Cu") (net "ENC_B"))
 (via (at 3.6211 18.5576) (size 0.6) (drill 0.3) (layers "F.Cu" "B.Cu") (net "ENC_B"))
 (segment (start 1.38 22.93) (end 3.621 20.689) (width 0.2) (layer "B.Cu") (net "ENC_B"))
 (segment (start 3.621 20.689) (end 3.621 18.5576) (width 0.2) (layer "B.Cu") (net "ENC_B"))
 (segment (start 3.621 18.5576) (end 3.6211 18.5576) (width 0.2) (layer "B.Cu") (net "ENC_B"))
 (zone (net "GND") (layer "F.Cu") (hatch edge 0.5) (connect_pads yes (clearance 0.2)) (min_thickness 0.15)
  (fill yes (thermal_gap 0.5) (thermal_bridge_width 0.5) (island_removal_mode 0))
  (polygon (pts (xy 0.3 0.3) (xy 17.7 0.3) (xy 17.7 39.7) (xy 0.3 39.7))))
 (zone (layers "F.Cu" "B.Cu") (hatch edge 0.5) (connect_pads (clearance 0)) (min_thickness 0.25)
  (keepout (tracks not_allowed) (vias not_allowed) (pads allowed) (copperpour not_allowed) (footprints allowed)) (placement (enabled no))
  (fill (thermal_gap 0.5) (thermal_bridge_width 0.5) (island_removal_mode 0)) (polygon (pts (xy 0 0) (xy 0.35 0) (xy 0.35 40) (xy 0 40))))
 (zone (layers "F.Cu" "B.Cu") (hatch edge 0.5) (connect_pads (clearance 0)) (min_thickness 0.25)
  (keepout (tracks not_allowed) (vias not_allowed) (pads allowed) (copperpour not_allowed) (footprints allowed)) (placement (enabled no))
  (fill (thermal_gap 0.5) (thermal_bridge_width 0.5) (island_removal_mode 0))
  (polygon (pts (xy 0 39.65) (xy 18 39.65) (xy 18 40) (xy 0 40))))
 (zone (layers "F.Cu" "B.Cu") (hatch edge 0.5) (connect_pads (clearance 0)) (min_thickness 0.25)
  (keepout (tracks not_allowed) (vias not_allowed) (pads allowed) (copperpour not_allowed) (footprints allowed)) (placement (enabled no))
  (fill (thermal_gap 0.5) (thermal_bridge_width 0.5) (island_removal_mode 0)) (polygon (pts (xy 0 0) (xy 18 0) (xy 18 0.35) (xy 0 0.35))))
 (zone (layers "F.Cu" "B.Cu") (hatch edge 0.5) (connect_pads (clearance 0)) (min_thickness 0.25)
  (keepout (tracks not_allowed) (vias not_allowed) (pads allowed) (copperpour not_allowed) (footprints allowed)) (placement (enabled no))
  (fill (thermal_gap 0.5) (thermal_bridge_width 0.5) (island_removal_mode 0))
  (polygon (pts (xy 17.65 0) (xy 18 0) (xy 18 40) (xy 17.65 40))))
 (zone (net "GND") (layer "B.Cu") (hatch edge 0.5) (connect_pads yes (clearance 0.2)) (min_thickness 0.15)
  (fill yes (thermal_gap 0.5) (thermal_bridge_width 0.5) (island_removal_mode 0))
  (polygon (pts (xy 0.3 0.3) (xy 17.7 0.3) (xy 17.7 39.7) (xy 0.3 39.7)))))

